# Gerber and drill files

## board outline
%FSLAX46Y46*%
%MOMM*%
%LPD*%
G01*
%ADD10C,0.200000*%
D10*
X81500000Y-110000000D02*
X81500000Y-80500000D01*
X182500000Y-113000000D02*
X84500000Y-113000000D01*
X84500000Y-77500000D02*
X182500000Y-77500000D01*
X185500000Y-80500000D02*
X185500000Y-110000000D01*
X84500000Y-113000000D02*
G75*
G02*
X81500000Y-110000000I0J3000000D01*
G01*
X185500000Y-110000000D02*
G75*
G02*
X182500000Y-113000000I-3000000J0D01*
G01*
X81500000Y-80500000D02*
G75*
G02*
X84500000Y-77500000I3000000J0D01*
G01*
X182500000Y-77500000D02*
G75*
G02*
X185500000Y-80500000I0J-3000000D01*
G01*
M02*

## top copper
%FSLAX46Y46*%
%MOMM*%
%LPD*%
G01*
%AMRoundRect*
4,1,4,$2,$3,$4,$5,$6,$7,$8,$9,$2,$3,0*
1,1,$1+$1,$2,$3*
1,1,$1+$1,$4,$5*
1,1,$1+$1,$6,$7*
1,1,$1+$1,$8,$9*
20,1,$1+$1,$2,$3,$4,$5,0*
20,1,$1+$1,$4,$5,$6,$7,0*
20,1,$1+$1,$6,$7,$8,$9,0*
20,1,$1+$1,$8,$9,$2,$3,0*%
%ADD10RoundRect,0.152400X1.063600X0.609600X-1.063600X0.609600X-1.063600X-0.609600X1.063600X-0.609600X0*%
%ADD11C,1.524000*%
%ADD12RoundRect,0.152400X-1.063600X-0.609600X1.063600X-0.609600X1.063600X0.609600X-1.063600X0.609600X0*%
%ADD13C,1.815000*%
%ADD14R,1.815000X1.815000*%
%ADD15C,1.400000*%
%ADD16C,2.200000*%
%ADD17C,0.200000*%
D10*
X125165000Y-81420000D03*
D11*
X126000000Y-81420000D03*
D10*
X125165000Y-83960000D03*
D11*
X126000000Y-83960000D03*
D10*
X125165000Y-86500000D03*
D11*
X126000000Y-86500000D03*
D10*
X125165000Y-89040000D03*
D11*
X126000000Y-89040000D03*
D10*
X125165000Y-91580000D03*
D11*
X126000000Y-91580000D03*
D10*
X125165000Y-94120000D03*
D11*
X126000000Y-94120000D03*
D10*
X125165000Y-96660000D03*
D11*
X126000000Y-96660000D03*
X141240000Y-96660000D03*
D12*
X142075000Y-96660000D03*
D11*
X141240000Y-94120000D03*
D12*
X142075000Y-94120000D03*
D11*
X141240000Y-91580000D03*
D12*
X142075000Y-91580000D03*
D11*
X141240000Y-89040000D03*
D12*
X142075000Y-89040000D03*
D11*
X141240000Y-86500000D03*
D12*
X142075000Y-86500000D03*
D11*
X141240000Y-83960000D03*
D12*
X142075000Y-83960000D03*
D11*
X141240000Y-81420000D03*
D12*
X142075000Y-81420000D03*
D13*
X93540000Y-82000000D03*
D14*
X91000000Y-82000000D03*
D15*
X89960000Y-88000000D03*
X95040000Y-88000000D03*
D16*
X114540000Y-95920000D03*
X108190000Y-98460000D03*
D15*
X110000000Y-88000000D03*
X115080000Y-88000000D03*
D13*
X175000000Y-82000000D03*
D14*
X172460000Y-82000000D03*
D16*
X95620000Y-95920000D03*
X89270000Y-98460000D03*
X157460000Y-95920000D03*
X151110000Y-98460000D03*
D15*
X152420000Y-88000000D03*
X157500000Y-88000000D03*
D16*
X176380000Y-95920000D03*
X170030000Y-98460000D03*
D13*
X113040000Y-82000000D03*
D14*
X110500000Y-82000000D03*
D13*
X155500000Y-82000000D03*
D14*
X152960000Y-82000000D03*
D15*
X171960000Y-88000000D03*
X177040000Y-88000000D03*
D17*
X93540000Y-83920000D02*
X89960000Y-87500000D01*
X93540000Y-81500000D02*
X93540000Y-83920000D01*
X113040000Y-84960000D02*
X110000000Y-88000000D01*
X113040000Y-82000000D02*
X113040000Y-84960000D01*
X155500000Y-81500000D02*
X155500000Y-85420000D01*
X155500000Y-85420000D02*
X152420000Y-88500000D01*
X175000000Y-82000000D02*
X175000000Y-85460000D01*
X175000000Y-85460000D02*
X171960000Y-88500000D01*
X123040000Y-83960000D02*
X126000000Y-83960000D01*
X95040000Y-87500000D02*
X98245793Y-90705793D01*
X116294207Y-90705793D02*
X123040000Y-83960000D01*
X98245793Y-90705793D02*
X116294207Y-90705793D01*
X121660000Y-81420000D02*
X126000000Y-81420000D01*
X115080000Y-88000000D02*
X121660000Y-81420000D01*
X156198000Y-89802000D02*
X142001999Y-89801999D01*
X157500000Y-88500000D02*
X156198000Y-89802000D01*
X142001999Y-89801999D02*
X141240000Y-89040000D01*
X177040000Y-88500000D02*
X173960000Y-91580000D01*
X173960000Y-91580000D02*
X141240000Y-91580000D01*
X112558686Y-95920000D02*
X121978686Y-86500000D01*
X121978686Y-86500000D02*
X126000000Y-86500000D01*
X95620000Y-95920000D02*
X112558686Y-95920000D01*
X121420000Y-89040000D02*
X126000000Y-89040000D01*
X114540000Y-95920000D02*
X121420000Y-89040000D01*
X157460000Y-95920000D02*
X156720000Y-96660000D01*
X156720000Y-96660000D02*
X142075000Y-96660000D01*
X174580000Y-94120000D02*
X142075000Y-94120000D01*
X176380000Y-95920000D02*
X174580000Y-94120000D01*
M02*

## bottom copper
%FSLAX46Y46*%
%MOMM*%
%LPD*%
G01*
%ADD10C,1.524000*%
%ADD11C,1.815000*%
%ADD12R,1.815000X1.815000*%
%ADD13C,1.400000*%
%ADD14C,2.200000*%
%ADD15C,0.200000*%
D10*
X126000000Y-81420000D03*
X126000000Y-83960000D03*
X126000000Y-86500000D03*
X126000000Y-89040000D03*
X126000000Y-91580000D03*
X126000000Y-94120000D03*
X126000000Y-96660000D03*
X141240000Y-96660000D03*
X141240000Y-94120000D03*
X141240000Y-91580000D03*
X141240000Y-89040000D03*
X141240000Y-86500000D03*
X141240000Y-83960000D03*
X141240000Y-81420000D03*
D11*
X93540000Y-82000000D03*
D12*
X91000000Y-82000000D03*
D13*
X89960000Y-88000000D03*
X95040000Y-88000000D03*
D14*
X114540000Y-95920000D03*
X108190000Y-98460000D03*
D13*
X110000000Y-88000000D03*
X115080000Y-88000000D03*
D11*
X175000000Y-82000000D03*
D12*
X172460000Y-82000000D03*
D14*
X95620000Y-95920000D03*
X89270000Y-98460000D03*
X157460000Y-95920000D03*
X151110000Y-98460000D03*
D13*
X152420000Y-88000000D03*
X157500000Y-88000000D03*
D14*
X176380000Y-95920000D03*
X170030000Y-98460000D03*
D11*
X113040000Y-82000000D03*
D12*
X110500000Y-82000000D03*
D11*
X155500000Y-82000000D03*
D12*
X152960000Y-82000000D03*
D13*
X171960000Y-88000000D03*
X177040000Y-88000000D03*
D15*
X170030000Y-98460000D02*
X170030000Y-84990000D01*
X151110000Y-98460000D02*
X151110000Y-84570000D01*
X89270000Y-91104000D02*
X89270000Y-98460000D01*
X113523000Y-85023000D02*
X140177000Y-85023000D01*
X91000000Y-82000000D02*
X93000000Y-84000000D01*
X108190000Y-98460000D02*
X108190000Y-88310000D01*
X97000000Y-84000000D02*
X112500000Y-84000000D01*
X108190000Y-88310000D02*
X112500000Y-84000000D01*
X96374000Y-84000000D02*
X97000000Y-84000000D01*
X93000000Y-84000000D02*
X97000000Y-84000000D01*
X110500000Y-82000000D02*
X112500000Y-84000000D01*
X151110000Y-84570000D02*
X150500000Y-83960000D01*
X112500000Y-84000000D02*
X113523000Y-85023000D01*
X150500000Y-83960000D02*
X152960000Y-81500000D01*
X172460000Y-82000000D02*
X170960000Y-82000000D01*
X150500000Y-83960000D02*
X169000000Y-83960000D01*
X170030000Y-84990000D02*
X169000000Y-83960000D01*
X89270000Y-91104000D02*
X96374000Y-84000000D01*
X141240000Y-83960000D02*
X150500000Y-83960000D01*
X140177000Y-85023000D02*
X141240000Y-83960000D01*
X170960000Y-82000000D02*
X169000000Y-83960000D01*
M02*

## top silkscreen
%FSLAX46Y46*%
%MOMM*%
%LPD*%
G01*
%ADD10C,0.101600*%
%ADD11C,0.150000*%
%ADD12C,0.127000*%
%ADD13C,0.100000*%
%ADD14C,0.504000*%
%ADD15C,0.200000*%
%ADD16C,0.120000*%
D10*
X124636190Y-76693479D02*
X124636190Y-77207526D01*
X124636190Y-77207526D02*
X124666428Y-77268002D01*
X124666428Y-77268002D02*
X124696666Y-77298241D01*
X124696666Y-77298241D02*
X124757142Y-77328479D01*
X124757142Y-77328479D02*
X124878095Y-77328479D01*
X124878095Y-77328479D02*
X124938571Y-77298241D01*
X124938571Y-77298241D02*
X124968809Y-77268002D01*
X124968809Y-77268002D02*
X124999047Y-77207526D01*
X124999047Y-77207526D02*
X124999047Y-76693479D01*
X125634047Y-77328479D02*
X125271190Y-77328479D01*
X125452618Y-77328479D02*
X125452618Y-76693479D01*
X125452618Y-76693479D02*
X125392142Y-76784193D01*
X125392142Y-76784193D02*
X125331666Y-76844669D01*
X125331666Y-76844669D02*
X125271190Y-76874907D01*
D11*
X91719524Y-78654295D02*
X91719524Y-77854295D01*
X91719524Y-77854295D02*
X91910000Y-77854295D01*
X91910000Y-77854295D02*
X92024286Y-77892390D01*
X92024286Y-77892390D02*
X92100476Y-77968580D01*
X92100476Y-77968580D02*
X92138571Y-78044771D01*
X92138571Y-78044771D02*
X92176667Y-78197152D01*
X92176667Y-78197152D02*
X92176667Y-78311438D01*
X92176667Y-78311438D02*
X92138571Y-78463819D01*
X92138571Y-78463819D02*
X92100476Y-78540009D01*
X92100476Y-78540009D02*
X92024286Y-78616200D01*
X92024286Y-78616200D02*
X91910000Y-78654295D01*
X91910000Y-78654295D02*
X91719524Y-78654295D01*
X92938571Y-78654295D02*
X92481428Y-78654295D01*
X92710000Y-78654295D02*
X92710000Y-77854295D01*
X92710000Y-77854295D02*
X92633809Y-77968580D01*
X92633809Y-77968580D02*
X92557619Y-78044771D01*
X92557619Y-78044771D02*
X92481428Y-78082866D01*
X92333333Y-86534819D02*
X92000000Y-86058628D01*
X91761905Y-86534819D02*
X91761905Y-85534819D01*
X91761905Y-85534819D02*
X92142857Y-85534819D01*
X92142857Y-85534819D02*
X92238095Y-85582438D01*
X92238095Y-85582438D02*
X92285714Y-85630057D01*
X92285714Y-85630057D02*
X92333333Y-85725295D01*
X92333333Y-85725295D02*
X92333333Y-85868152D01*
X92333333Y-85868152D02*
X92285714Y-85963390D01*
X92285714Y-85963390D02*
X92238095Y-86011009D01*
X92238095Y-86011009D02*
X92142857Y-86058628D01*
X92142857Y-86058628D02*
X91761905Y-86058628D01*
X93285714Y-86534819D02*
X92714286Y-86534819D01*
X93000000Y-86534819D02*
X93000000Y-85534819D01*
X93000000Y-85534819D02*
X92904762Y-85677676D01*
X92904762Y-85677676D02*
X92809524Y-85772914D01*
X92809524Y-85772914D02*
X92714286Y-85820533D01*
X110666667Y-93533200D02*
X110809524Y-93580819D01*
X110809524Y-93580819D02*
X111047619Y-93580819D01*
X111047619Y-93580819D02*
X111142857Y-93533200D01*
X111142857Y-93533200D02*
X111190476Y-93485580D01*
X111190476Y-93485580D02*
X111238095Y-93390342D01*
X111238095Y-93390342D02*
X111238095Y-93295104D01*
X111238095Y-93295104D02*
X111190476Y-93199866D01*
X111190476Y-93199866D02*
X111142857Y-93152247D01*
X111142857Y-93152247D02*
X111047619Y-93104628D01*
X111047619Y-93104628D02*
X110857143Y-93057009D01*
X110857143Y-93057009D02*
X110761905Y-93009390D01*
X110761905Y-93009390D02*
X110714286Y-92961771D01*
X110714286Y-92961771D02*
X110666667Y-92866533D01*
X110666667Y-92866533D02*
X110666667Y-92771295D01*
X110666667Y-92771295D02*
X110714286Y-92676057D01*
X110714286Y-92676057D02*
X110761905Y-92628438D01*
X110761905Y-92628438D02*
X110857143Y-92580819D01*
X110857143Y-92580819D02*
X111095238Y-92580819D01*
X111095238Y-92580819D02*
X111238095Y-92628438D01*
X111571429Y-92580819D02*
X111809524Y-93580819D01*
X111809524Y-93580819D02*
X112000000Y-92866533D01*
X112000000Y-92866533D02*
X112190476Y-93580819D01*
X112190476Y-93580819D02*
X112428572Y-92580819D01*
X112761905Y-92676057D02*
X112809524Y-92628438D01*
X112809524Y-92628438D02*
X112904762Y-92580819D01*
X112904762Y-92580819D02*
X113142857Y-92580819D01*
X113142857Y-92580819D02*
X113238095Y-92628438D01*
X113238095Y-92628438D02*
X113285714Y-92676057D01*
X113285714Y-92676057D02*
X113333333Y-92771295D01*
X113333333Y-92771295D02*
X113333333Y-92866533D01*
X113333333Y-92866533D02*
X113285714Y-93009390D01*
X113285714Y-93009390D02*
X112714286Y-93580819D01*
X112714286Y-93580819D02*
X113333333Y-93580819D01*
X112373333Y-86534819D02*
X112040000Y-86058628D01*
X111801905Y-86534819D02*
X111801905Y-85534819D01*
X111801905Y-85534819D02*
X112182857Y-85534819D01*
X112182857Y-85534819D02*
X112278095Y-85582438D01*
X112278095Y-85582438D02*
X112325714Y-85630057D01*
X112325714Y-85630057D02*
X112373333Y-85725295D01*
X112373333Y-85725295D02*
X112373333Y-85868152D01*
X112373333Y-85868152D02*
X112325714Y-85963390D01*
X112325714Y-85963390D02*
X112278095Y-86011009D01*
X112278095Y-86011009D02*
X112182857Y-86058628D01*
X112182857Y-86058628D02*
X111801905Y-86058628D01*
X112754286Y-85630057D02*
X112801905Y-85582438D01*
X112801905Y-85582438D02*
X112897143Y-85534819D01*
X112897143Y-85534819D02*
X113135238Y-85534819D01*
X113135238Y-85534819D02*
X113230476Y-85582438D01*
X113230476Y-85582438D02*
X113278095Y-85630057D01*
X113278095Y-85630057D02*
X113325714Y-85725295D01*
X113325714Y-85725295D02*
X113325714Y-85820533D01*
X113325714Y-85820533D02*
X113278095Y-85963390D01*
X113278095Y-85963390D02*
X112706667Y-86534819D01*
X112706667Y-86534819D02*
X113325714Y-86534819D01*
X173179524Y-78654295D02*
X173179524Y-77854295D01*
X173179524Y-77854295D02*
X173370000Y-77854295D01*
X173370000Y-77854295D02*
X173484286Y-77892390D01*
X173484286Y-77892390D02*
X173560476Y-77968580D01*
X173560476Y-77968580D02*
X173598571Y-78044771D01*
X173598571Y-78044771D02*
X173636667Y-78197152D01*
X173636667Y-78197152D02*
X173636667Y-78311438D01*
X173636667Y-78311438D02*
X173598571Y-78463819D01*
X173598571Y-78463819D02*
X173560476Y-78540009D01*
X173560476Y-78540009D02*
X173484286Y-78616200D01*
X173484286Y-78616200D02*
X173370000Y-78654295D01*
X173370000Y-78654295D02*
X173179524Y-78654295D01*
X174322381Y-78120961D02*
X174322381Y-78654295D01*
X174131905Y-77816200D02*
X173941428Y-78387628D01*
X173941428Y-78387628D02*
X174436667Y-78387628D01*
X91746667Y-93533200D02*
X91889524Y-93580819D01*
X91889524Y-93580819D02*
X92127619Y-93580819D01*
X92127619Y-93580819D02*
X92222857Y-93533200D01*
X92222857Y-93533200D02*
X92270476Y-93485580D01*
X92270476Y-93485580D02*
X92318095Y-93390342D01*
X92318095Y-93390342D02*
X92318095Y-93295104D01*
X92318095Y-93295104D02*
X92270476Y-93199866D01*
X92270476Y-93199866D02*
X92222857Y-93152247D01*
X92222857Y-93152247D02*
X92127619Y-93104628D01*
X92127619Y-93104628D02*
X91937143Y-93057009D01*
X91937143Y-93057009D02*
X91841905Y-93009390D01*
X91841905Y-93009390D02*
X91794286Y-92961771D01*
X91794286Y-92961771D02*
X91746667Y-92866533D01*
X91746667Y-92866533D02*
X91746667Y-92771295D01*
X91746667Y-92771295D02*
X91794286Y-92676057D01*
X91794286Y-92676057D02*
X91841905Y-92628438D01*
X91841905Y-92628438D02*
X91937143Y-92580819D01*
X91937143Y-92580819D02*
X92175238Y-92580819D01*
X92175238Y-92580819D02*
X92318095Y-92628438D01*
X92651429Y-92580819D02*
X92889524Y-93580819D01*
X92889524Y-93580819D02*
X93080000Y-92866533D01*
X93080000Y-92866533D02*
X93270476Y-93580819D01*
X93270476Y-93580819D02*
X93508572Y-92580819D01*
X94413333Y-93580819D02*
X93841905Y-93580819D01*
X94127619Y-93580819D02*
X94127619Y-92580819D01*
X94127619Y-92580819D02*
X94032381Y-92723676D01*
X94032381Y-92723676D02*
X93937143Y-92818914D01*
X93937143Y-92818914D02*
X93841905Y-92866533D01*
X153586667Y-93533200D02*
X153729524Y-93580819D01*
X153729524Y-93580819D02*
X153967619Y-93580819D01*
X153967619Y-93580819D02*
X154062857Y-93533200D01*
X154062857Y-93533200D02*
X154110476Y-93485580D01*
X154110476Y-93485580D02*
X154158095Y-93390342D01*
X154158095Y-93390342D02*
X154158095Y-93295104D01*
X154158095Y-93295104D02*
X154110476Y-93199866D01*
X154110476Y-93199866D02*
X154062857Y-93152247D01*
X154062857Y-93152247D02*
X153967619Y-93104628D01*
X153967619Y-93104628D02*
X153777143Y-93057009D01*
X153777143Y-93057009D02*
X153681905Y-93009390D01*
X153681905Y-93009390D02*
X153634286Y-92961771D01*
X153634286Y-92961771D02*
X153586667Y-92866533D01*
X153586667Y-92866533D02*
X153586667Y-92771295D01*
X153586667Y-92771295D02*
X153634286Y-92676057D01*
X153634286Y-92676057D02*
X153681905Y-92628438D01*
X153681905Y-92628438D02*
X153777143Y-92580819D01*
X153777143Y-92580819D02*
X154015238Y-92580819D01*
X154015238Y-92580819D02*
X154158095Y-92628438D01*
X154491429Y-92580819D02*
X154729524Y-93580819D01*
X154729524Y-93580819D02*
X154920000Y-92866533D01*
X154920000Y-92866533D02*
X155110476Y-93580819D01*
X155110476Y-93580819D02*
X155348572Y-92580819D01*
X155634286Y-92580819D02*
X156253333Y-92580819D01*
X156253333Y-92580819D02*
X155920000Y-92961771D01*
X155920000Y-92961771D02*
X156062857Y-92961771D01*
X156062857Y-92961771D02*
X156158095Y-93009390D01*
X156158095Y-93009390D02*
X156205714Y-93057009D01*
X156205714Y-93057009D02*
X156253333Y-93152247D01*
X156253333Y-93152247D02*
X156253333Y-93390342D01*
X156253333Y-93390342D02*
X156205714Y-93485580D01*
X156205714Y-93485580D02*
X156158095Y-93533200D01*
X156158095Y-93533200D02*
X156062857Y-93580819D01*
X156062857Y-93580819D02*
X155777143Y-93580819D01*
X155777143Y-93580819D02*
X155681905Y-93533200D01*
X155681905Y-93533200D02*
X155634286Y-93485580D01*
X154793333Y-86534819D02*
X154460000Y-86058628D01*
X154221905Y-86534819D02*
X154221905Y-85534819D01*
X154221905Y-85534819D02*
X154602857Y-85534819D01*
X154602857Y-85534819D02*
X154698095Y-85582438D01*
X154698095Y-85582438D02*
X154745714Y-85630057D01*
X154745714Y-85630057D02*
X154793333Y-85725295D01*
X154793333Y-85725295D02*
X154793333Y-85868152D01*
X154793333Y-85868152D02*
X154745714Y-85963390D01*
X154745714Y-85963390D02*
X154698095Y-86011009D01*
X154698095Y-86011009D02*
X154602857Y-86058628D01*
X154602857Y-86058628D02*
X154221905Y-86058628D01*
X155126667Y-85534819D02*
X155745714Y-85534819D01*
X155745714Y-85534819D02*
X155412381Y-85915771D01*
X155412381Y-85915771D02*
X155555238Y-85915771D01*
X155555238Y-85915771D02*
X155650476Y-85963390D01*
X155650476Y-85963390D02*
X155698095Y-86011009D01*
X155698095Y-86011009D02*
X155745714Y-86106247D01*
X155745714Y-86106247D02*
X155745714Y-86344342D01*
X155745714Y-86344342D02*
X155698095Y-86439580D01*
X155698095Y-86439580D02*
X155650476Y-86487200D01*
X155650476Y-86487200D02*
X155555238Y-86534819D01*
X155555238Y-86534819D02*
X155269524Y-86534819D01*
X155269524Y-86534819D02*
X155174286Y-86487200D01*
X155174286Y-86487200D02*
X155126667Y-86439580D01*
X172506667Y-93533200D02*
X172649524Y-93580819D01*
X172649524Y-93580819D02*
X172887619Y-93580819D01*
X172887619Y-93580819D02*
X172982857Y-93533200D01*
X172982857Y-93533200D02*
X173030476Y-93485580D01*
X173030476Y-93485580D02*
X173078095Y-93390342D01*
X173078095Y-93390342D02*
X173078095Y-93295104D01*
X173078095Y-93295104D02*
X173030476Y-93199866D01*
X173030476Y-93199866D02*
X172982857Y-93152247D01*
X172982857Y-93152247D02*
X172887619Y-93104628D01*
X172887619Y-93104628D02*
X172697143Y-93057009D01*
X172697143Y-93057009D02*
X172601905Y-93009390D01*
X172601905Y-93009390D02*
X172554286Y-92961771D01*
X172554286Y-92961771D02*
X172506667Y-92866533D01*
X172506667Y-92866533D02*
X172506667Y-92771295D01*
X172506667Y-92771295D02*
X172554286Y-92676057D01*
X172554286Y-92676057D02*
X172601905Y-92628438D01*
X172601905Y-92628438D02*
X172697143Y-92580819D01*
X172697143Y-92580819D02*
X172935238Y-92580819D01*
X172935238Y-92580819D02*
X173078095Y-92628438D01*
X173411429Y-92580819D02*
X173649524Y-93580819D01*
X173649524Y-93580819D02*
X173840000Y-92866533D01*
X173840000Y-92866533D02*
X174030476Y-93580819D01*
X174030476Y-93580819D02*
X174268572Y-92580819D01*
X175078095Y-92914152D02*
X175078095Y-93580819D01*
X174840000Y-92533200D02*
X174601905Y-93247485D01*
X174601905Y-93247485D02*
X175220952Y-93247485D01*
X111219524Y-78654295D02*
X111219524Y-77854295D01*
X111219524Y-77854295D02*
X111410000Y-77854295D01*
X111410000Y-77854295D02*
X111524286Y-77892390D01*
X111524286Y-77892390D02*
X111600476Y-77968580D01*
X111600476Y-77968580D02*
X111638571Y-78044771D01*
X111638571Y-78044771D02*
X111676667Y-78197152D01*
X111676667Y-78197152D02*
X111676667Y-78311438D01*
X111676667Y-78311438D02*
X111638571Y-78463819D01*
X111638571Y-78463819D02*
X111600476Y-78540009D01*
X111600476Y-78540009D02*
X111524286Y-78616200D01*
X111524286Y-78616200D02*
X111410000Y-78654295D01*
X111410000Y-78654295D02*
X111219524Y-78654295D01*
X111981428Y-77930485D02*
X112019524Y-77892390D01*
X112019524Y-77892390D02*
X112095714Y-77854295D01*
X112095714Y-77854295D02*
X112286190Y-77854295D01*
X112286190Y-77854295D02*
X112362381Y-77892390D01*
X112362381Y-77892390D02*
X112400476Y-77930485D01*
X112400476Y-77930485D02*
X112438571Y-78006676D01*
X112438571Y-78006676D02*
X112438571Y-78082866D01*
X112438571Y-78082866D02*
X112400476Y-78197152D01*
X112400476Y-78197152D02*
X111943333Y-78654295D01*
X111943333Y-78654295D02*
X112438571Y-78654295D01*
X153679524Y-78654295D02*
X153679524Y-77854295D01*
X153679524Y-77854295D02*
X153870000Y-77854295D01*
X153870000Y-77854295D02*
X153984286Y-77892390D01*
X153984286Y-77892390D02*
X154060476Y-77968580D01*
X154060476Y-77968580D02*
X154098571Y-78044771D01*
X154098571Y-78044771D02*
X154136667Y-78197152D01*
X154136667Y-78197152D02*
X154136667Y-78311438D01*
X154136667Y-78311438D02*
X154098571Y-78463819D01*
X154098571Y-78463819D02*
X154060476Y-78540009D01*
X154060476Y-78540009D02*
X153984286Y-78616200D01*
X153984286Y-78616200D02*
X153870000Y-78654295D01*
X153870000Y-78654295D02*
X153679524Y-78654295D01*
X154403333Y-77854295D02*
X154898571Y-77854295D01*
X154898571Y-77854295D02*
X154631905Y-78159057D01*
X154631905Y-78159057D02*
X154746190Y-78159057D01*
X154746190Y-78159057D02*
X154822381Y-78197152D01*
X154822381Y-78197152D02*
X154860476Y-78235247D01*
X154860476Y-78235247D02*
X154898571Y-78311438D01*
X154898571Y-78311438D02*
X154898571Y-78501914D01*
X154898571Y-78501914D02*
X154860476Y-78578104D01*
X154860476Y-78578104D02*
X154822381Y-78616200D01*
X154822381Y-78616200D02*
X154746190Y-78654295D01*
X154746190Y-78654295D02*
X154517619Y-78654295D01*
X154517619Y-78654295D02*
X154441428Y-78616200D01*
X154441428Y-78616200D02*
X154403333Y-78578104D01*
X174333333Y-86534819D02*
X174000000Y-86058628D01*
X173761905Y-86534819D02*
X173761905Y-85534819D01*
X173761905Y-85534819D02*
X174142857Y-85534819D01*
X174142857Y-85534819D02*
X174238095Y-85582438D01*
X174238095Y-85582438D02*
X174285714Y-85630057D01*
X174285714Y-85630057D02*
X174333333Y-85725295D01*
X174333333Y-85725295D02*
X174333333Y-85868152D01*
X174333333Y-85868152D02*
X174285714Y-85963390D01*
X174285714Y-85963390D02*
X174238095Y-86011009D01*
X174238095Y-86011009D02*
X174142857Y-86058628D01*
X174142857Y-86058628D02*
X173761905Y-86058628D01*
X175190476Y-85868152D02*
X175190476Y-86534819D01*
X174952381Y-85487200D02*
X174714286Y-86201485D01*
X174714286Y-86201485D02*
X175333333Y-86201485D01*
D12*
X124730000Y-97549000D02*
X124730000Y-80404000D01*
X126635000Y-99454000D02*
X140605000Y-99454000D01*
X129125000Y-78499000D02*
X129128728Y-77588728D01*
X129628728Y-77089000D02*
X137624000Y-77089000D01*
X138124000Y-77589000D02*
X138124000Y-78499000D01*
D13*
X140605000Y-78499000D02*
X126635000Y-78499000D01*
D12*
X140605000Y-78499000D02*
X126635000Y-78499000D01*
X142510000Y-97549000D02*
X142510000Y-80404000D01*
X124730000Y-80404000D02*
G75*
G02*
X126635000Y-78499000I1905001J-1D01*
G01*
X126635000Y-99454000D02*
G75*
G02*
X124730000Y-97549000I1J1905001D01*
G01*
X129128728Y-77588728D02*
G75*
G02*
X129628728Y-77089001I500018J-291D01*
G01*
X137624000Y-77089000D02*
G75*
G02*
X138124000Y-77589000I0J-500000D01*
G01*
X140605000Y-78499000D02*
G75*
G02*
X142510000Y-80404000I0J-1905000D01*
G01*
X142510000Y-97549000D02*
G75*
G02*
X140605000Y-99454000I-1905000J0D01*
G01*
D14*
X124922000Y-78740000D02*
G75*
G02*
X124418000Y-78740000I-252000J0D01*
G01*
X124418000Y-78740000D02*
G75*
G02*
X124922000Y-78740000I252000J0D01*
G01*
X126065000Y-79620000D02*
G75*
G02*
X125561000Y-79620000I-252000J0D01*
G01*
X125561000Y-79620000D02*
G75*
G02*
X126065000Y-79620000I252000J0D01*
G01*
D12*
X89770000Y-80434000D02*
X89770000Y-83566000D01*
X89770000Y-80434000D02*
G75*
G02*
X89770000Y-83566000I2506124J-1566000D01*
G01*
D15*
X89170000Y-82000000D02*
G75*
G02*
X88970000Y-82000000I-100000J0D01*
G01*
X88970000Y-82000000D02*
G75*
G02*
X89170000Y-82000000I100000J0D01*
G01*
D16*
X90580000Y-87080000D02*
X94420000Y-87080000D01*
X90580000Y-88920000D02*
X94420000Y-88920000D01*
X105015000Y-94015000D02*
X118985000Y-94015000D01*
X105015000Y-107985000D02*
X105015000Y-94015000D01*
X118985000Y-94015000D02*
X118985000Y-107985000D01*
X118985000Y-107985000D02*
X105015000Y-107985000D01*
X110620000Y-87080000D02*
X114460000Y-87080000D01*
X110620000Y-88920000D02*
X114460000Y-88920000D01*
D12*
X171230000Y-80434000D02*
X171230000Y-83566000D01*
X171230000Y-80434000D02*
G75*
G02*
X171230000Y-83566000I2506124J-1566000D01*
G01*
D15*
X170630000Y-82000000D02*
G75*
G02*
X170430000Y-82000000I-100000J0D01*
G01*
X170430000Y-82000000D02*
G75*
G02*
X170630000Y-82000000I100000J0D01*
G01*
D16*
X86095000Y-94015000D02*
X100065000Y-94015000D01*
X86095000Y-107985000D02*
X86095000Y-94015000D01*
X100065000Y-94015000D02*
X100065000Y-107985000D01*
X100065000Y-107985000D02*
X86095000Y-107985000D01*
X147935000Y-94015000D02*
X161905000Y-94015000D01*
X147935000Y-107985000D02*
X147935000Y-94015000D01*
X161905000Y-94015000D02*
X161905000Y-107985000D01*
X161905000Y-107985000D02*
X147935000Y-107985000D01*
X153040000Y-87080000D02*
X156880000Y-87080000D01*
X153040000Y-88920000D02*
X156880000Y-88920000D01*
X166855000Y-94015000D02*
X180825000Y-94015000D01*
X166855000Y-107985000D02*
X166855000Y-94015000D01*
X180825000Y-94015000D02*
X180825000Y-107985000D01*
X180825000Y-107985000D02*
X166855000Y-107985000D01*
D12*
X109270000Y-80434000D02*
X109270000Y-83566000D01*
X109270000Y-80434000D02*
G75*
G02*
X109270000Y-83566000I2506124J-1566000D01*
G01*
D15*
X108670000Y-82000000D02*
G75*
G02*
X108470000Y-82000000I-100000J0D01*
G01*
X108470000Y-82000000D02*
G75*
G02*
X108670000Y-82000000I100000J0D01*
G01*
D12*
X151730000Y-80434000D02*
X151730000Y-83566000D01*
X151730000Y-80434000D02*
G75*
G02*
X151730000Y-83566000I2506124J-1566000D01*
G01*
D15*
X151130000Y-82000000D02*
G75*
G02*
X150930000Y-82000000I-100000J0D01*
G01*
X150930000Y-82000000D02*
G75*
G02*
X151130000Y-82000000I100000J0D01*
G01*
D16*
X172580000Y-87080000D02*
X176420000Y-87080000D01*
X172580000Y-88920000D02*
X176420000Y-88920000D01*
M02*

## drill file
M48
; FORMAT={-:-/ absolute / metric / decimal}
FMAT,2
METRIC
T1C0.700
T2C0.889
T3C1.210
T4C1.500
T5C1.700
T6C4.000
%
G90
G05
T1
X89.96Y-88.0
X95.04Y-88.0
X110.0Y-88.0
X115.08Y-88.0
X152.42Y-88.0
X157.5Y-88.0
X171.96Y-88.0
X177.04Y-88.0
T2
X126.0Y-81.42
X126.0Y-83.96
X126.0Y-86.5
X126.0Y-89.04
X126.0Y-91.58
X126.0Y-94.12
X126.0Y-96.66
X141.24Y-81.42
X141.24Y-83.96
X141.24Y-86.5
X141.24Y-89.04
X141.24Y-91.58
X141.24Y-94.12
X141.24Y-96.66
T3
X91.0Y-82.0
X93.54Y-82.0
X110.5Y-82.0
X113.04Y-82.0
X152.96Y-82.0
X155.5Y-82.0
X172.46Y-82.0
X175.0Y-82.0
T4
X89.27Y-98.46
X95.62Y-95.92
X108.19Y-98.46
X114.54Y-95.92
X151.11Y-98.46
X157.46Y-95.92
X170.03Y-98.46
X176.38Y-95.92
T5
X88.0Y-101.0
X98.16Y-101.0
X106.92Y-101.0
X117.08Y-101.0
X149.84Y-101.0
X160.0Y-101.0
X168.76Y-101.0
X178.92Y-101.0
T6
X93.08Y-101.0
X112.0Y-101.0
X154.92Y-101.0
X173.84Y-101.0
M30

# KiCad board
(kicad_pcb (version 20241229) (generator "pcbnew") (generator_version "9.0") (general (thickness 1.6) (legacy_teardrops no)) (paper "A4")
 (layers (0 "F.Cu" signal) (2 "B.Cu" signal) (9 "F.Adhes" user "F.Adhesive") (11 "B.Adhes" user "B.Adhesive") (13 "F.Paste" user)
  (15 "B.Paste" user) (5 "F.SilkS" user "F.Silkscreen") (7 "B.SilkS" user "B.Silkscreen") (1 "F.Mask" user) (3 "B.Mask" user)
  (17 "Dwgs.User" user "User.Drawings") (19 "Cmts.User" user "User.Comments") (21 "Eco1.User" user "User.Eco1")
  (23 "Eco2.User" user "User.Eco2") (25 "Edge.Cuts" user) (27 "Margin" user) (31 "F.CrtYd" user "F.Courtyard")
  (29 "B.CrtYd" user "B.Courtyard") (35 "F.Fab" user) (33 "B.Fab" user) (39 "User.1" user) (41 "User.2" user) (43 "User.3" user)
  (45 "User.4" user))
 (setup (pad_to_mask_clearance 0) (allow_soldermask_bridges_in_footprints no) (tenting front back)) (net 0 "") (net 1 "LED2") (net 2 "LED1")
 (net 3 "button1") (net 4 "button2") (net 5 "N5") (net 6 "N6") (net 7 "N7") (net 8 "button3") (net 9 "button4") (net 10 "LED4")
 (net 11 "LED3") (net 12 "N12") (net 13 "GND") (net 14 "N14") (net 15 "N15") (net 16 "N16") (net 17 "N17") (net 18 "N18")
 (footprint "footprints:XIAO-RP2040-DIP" (layer "F.Cu") (at 133.62 89.04)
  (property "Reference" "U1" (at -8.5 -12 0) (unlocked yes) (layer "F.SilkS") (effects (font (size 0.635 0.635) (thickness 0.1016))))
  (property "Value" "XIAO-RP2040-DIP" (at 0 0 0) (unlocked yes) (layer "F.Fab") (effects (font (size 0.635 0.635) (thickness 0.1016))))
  (fp_line (start -8.89 8.509) (end -8.89 -8.636) (stroke (width 0.127) (type solid)) (layer "F.SilkS"))
  (fp_line (start -6.985 10.414) (end 6.985 10.414) (stroke (width 0.127) (type solid)) (layer "F.SilkS"))
  (fp_line (start -4.495 -10.541) (end -4.491272 -11.451272) (stroke (width 0.127) (type solid)) (layer "F.SilkS"))
  (fp_line (start -3.991272 -11.951) (end 4.004 -11.951) (stroke (width 0.127) (type solid)) (layer "F.SilkS"))
  (fp_line (start 4.504 -11.451) (end 4.504 -10.541) (stroke (width 0.127) (type solid)) (layer "F.SilkS"))
  (fp_line (start 6.985 -10.541) (end -6.985 -10.541) (stroke (width 0.1) (type solid)) (layer "F.SilkS"))
  (fp_line (start 6.985 -10.541) (end -6.985 -10.541) (stroke (width 0.127) (type solid)) (layer "F.SilkS"))
  (fp_line (start 8.89 8.509) (end 8.89 -8.636) (stroke (width 0.127) (type solid)) (layer "F.SilkS"))
  (fp_arc (start -8.89 -8.636) (mid -8.332038 -9.983038) (end -6.985 -10.541) (stroke (width 0.127) (type solid)) (layer "F.SilkS"))
  (fp_arc (start -6.985 10.414) (mid -8.332038 9.856038) (end -8.89 8.509) (stroke (width 0.127) (type solid)) (layer "F.SilkS"))
  (fp_arc (start -4.491272 -11.451272) (mid -4.344728 -11.80464) (end -3.991272 -11.951) (stroke (width 0.127) (type default))
   (layer "F.SilkS"))
  (fp_arc (start 4.004 -11.951) (mid 4.357553 -11.804553) (end 4.504 -11.451) (stroke (width 0.127) (type default)) (layer "F.SilkS"))
  (fp_arc (start 6.985 -10.541) (mid 8.332038 -9.983038) (end 8.89 -8.636) (stroke (width 0.127) (type solid)) (layer "F.SilkS"))
  (fp_arc (start 8.89 8.509) (mid 8.332038 9.856038) (end 6.985 10.414) (stroke (width 0.127) (type solid)) (layer "F.SilkS"))
  (fp_circle (center -8.95 -10.3) (end -8.95 -10.554) (stroke (width 0.5) (type solid)) (fill yes) (layer "F.SilkS"))
  (fp_circle (center -7.807 -9.42) (end -7.807 -9.674) (stroke (width 0.5) (type solid)) (fill yes) (layer "F.SilkS"))
  (pad "1" smd roundrect (at -8.455 -7.62 180) (size 2.432 1.524) (layers "F.Cu" "F.Mask") (roundrect_rratio 0.1) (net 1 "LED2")
   (thermal_bridge_angle 45))
  (pad "1" thru_hole circle (at -7.62 -7.62 180) (size 1.524 1.524) (drill 0.889) (layers "*.Cu" "*.Mask") (remove_unused_layers no)
   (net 1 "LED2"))
  (pad "2" smd roundrect (at -8.455 -5.08 180) (size 2.432 1.524) (layers "F.Cu" "F.Mask") (roundrect_rratio 0.1) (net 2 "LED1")
   (thermal_bridge_angle 45))
  (pad "2" thru_hole circle (at -7.62 -5.08 180) (size 1.524 1.524) (drill 0.889) (layers "*.Cu" "*.Mask") (remove_unused_layers no)
   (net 2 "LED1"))
  (pad "3" smd roundrect (at -8.455 -2.54 180) (size 2.432 1.524) (layers "F.Cu" "F.Mask") (roundrect_rratio 0.1) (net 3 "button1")
   (thermal_bridge_angle 45))
  (pad "3" thru_hole circle (at -7.62 -2.54 180) (size 1.524 1.524) (drill 0.889) (layers "*.Cu" "*.Mask") (remove_unused_layers no)
   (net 3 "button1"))
  (pad "4" smd roundrect (at -8.455 0 180) (size 2.432 1.524) (layers "F.Cu" "F.Mask") (roundrect_rratio 0.1) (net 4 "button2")
   (thermal_bridge_angle 45))
  (pad "4" thru_hole circle (at -7.62 0 180) (size 1.524 1.524) (drill 0.889) (layers "*.Cu" "*.Mask") (remove_unused_layers no)
   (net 4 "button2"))
  (pad "5" smd roundrect (at -8.455 2.54 180) (size 2.432 1.524) (layers "F.Cu" "F.Mask") (roundrect_rratio 0.1) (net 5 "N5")
   (thermal_bridge_angle 45))
  (pad "5" thru_hole circle (at -7.62 2.54 180) (size 1.524 1.524) (drill 0.889) (layers "*.Cu" "*.Mask") (remove_unused_layers no)
   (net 5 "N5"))
  (pad "6" smd roundrect (at -8.455 5.08 180) (size 2.432 1.524) (layers "F.Cu" "F.Mask") (roundrect_rratio 0.1) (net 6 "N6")
   (thermal_bridge_angle 45))
  (pad "6" thru_hole circle (at -7.62 5.08 180) (size 1.524 1.524) (drill 0.889) (layers "*.Cu" "*.Mask") (remove_unused_layers no)
   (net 6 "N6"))
  (pad "7" smd roundrect (at -8.455 7.62 180) (size 2.432 1.524) (layers "F.Cu" "F.Mask") (roundrect_rratio 0.1) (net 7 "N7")
   (thermal_bridge_angle 45))
  (pad "7" thru_hole circle (at -7.62 7.62 180) (size 1.524 1.524) (drill 0.889) (layers "*.Cu" "*.Mask") (remove_unused_layers no)
   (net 7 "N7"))
  (pad "8" thru_hole circle (at 7.62 7.62) (size 1.524 1.524) (drill 0.889) (layers "*.Cu" "*.Mask") (remove_unused_layers no)
   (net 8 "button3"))
  (pad "8" smd roundrect (at 8.455 7.62) (size 2.432 1.524) (layers "F.Cu" "F.Mask") (roundrect_rratio 0.1) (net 8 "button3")
   (thermal_bridge_angle 45))
  (pad "9" thru_hole circle (at 7.62 5.08) (size 1.524 1.524) (drill 0.889) (layers "*.Cu" "*.Mask") (remove_unused_layers no)
   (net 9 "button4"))
  (pad "9" smd roundrect (at 8.455 5.08) (size 2.432 1.524) (layers "F.Cu" "F.Mask") (roundrect_rratio 0.1) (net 9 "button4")
   (thermal_bridge_angle 45))
  (pad "10" thru_hole circle (at 7.62 2.54) (size 1.524 1.524) (drill 0.889) (layers "*.Cu" "*.Mask") (remove_unused_layers no)
   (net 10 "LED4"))
  (pad "10" smd roundrect (at 8.455 2.54) (size 2.432 1.524) (layers "F.Cu" "F.Mask") (roundrect_rratio 0.1) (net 10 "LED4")
   (thermal_bridge_angle 45))
  (pad "11" thru_hole circle (at 7.62 0) (size 1.524 1.524) (drill 0.889) (layers "*.Cu" "*.Mask") (remove_unused_layers no) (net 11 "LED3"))
  (pad "11" smd roundrect (at 8.455 0) (size 2.432 1.524) (layers "F.Cu" "F.Mask") (roundrect_rratio 0.1) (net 11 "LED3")
   (thermal_bridge_angle 45))
  (pad "12" thru_hole circle (at 7.62 -2.54) (size 1.524 1.524) (drill 0.889) (layers "*.Cu" "*.Mask") (remove_unused_layers no)
   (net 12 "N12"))
  (pad "12" smd roundrect (at 8.455 -2.54) (size 2.432 1.524) (layers "F.Cu" "F.Mask") (roundrect_rratio 0.1) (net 12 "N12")
   (thermal_bridge_angle 45))
  (pad "13" thru_hole circle (at 7.62 -5.08) (size 1.524 1.524) (drill 0.889) (layers "*.Cu" "*.Mask") (remove_unused_layers no)
   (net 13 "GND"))
  (pad "13" smd roundrect (at 8.455 -5.08) (size 2.432 1.524) (layers "F.Cu" "F.Mask") (roundrect_rratio 0.1) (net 13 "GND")
   (thermal_bridge_angle 45))
  (pad "14" thru_hole circle (at 7.62 -7.62) (size 1.524 1.524) (drill 0.889) (layers "*.Cu" "*.Mask") (remove_unused_layers no)
   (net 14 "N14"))
  (pad "14" smd roundrect (at 8.455 -7.62) (size 2.432 1.524) (layers "F.Cu" "F.Mask") (roundrect_rratio 0.1) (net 14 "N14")
   (thermal_bridge_angle 45)))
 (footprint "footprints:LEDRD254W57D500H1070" (layer "F.Cu") (at 92.27 82)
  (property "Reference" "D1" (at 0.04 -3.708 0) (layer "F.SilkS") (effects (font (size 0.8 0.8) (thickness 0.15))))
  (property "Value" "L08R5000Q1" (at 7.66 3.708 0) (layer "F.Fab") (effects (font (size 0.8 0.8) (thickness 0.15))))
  (fp_line (start -2.5 -1.566) (end -2.5 1.566) (stroke (width 0.127) (type solid)) (layer "F.SilkS"))
  (fp_arc (start -2.5 -1.566) (mid 2.961291 0) (end -2.5 1.566) (stroke (width 0.127) (type solid)) (layer "F.SilkS"))
  (fp_circle (center -3.2 0) (end -3.1 0) (stroke (width 0.2) (type solid)) (fill no) (layer "F.SilkS"))
  (pad "A" thru_hole circle (at 1.27 0) (size 1.815 1.815) (drill 1.21) (layers "*.Cu" "*.Mask") (remove_unused_layers no) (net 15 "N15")
   (solder_mask_margin 0.102))
  (pad "C" thru_hole rect (at -1.27 0) (size 1.815 1.815) (drill 1.21) (layers "*.Cu" "*.Mask") (remove_unused_layers no) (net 13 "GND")
   (solder_mask_margin 0.102)))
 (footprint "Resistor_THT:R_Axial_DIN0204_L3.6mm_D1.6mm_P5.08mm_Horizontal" (layer "F.Cu") (at 89.96 88)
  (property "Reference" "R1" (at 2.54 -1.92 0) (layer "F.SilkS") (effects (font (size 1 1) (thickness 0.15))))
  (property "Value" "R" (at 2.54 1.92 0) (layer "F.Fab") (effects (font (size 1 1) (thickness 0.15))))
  (fp_line (start 0.62 -0.92) (end 4.46 -0.92) (stroke (width 0.12) (type solid)) (layer "F.SilkS"))
  (fp_line (start 0.62 0.92) (end 4.46 0.92) (stroke (width 0.12) (type solid)) (layer "F.SilkS"))
  (pad "1" thru_hole circle (at 0 0) (size 1.4 1.4) (drill 0.7) (layers "*.Cu" "*.Mask") (remove_unused_layers no) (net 15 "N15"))
  (pad "2" thru_hole circle (at 5.08 0) (size 1.4 1.4) (drill 0.7) (layers "*.Cu" "*.Mask") (remove_unused_layers no) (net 2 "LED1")))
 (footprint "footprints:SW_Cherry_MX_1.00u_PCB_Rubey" (layer "F.Cu") (at 114.54 95.92)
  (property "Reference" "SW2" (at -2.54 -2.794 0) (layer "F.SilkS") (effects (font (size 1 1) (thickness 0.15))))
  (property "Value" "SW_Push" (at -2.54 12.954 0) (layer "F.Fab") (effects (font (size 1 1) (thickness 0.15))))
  (fp_line (start -9.525 -1.905) (end 4.445 -1.905) (stroke (width 0.12) (type solid)) (layer "F.SilkS"))
  (fp_line (start -9.525 12.065) (end -9.525 -1.905) (stroke (width 0.12) (type solid)) (layer "F.SilkS"))
  (fp_line (start 4.445 -1.905) (end 4.445 12.065) (stroke (width 0.12) (type solid)) (layer "F.SilkS"))
  (fp_line (start 4.445 12.065) (end -9.525 12.065) (stroke (width 0.12) (type solid)) (layer "F.SilkS"))
  (pad "" np_thru_hole circle (at -7.62 5.08) (size 1.7 1.7) (drill 1.7) (layers "*.Cu" "*.Mask"))
  (pad "" np_thru_hole circle (at -2.54 5.08) (size 4 4) (drill 4) (layers "*.Cu" "*.Mask"))
  (pad "" np_thru_hole circle (at 2.54 5.08) (size 1.7 1.7) (drill 1.7) (layers "*.Cu" "*.Mask"))
  (pad "1" thru_hole circle (at 0 0) (size 2.2 2.2) (drill 1.5) (layers "*.Cu" "*.Mask") (remove_unused_layers no) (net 4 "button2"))
  (pad "2" thru_hole circle (at -6.35 2.54) (size 2.2 2.2) (drill 1.5) (layers "*.Cu" "*.Mask") (remove_unused_layers no) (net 13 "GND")))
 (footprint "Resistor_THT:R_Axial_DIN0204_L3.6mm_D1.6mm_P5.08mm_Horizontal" (layer "F.Cu") (at 110 88)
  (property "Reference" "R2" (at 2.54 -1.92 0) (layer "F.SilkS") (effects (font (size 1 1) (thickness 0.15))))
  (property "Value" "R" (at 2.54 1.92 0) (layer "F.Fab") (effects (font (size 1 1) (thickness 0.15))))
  (fp_line (start 0.62 -0.92) (end 4.46 -0.92) (stroke (width 0.12) (type solid)) (layer "F.SilkS"))
  (fp_line (start 0.62 0.92) (end 4.46 0.92) (stroke (width 0.12) (type solid)) (layer "F.SilkS"))
  (pad "1" thru_hole circle (at 0 0) (size 1.4 1.4) (drill 0.7) (layers "*.Cu" "*.Mask") (remove_unused_layers no) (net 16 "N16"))
  (pad "2" thru_hole circle (at 5.08 0) (size 1.4 1.4) (drill 0.7) (layers "*.Cu" "*.Mask") (remove_unused_layers no) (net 1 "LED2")))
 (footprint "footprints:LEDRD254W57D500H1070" (layer "F.Cu") (at 173.73 82)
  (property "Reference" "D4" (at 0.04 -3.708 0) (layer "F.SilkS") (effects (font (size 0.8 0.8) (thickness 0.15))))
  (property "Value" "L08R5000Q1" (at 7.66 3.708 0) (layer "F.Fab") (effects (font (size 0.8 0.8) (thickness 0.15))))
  (fp_line (start -2.5 -1.566) (end -2.5 1.566) (stroke (width 0.127) (type solid)) (layer "F.SilkS"))
  (fp_arc (start -2.5 -1.566) (mid 2.961291 0) (end -2.5 1.566) (stroke (width 0.127) (type solid)) (layer "F.SilkS"))
  (fp_circle (center -3.2 0) (end -3.1 0) (stroke (width 0.2) (type solid)) (fill no) (layer "F.SilkS"))
  (pad "A" thru_hole circle (at 1.27 0) (size 1.815 1.815) (drill 1.21) (layers "*.Cu" "*.Mask") (remove_unused_layers no) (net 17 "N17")
   (solder_mask_margin 0.102))
  (pad "C" thru_hole rect (at -1.27 0) (size 1.815 1.815) (drill 1.21) (layers "*.Cu" "*.Mask") (remove_unused_layers no) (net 13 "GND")
   (solder_mask_margin 0.102)))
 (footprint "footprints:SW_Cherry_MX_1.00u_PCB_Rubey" (layer "F.Cu") (at 95.62 95.92)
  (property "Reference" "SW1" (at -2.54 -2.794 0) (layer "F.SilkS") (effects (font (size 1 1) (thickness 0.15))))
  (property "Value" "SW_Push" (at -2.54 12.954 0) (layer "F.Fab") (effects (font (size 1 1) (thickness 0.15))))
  (fp_line (start -9.525 -1.905) (end 4.445 -1.905) (stroke (width 0.12) (type solid)) (layer "F.SilkS"))
  (fp_line (start -9.525 12.065) (end -9.525 -1.905) (stroke (width 0.12) (type solid)) (layer "F.SilkS"))
  (fp_line (start 4.445 -1.905) (end 4.445 12.065) (stroke (width 0.12) (type solid)) (layer "F.SilkS"))
  (fp_line (start 4.445 12.065) (end -9.525 12.065) (stroke (width 0.12) (type solid)) (layer "F.SilkS"))
  (pad "" np_thru_hole circle (at -7.62 5.08) (size 1.7 1.7) (drill 1.7) (layers "*.Cu" "*.Mask"))
  (pad "" np_thru_hole circle (at -2.54 5.08) (size 4 4) (drill 4) (layers "*.Cu" "*.Mask"))
  (pad "" np_thru_hole circle (at 2.54 5.08) (size 1.7 1.7) (drill 1.7) (layers "*.Cu" "*.Mask"))
  (pad "1" thru_hole circle (at 0 0) (size 2.2 2.2) (drill 1.5) (layers "*.Cu" "*.Mask") (remove_unused_layers no) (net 3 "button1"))
  (pad "2" thru_hole circle (at -6.35 2.54) (size 2.2 2.2) (drill 1.5) (layers "*.Cu" "*.Mask") (remove_unused_layers no) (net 13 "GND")))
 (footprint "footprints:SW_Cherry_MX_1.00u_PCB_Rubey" (layer "F.Cu") (at 157.46 95.92)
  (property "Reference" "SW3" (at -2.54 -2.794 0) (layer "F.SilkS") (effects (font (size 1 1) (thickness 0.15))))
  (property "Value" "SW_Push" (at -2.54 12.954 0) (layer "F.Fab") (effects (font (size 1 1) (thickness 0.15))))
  (fp_line (start -9.525 -1.905) (end 4.445 -1.905) (stroke (width 0.12) (type solid)) (layer "F.SilkS"))
  (fp_line (start -9.525 12.065) (end -9.525 -1.905) (stroke (width 0.12) (type solid)) (layer "F.SilkS"))
  (fp_line (start 4.445 -1.905) (end 4.445 12.065) (stroke (width 0.12) (type solid)) (layer "F.SilkS"))
  (fp_line (start 4.445 12.065) (end -9.525 12.065) (stroke (width 0.12) (type solid)) (layer "F.SilkS"))
  (pad "" np_thru_hole circle (at -7.62 5.08) (size 1.7 1.7) (drill 1.7) (layers "*.Cu" "*.Mask"))
  (pad "" np_thru_hole circle (at -2.54 5.08) (size 4 4) (drill 4) (layers "*.Cu" "*.Mask"))
  (pad "" np_thru_hole circle (at 2.54 5.08) (size 1.7 1.7) (drill 1.7) (layers "*.Cu" "*.Mask"))
  (pad "1" thru_hole circle (at 0 0) (size 2.2 2.2) (drill 1.5) (layers "*.Cu" "*.Mask") (remove_unused_layers no) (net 8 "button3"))
  (pad "2" thru_hole circle (at -6.35 2.54) (size 2.2 2.2) (drill 1.5) (layers "*.Cu" "*.Mask") (remove_unused_layers no) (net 13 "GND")))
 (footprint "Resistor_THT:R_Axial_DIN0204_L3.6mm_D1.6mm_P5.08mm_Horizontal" (layer "F.Cu") (at 152.42 88)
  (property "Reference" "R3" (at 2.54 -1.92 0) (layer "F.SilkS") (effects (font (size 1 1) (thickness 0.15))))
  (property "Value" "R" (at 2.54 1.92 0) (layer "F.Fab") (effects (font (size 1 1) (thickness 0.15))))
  (fp_line (start 0.62 -0.92) (end 4.46 -0.92) (stroke (width 0.12) (type solid)) (layer "F.SilkS"))
  (fp_line (start 0.62 0.92) (end 4.46 0.92) (stroke (width 0.12) (type solid)) (layer "F.SilkS"))
  (pad "1" thru_hole circle (at 0 0) (size 1.4 1.4) (drill 0.7) (layers "*.Cu" "*.Mask") (remove_unused_layers no) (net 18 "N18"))
  (pad "2" thru_hole circle (at 5.08 0) (size 1.4 1.4) (drill 0.7) (layers "*.Cu" "*.Mask") (remove_unused_layers no) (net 11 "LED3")))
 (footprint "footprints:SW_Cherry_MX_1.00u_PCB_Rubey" (layer "F.Cu") (at 176.38 95.92)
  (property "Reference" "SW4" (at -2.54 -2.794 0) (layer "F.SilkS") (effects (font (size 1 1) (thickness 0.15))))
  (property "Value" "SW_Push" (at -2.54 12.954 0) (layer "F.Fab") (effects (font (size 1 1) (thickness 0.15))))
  (fp_line (start -9.525 -1.905) (end 4.445 -1.905) (stroke (width 0.12) (type solid)) (layer "F.SilkS"))
  (fp_line (start -9.525 12.065) (end -9.525 -1.905) (stroke (width 0.12) (type solid)) (layer "F.SilkS"))
  (fp_line (start 4.445 -1.905) (end 4.445 12.065) (stroke (width 0.12) (type solid)) (layer "F.SilkS"))
  (fp_line (start 4.445 12.065) (end -9.525 12.065) (stroke (width 0.12) (type solid)) (layer "F.SilkS"))
  (pad "" np_thru_hole circle (at -7.62 5.08) (size 1.7 1.7) (drill 1.7) (layers "*.Cu" "*.Mask"))
  (pad "" np_thru_hole circle (at -2.54 5.08) (size 4 4) (drill 4) (layers "*.Cu" "*.Mask"))
  (pad "" np_thru_hole circle (at 2.54 5.08) (size 1.7 1.7) (drill 1.7) (layers "*.Cu" "*.Mask"))
  (pad "1" thru_hole circle (at 0 0) (size 2.2 2.2) (drill 1.5) (layers "*.Cu" "*.Mask") (remove_unused_layers no) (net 9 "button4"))
  (pad "2" thru_hole circle (at -6.35 2.54) (size 2.2 2.2) (drill 1.5) (layers "*.Cu" "*.Mask") (remove_unused_layers no) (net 13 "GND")))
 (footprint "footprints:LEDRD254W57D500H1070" (layer "F.Cu") (at 111.77 82)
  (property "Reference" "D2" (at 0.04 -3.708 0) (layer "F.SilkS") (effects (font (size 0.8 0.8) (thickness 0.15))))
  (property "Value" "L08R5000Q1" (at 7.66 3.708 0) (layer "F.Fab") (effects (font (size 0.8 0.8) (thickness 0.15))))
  (fp_line (start -2.5 -1.566) (end -2.5 1.566) (stroke (width 0.127) (type solid)) (layer "F.SilkS"))
  (fp_arc (start -2.5 -1.566) (mid 2.961291 0) (end -2.5 1.566) (stroke (width 0.127) (type solid)) (layer "F.SilkS"))
  (fp_circle (center -3.2 0) (end -3.1 0) (stroke (width 0.2) (type solid)) (fill no) (layer "F.SilkS"))
  (pad "A" thru_hole circle (at 1.27 0) (size 1.815 1.815) (drill 1.21) (layers "*.Cu" "*.Mask") (remove_unused_layers no) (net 16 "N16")
   (solder_mask_margin 0.102))
  (pad "C" thru_hole rect (at -1.27 0) (size 1.815 1.815) (drill 1.21) (layers "*.Cu" "*.Mask") (remove_unused_layers no) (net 13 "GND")
   (solder_mask_margin 0.102)))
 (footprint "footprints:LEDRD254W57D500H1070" (layer "F.Cu") (at 154.23 82)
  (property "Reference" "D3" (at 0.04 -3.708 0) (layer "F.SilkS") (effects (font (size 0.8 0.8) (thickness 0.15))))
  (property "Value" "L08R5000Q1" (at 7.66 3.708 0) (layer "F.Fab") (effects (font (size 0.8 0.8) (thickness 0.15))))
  (fp_line (start -2.5 -1.566) (end -2.5 1.566) (stroke (width 0.127) (type solid)) (layer "F.SilkS"))
  (fp_arc (start -2.5 -1.566) (mid 2.961291 0) (end -2.5 1.566) (stroke (width 0.127) (type solid)) (layer "F.SilkS"))
  (fp_circle (center -3.2 0) (end -3.1 0) (stroke (width 0.2) (type solid)) (fill no) (layer "F.SilkS"))
  (pad "A" thru_hole circle (at 1.27 0) (size 1.815 1.815) (drill 1.21) (layers "*.Cu" "*.Mask") (remove_unused_layers no) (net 18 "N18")
   (solder_mask_margin 0.102))
  (pad "C" thru_hole rect (at -1.27 0) (size 1.815 1.815) (drill 1.21) (layers "*.Cu" "*.Mask") (remove_unused_layers no) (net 13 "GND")
   (solder_mask_margin 0.102)))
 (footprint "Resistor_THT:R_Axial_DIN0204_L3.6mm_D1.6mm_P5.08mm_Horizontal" (layer "F.Cu") (at 171.96 88)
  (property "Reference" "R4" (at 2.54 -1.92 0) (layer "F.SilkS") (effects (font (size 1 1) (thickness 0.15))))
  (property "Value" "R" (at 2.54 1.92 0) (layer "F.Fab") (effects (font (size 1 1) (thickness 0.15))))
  (fp_line (start 0.62 -0.92) (end 4.46 -0.92) (stroke (width 0.12) (type solid)) (layer "F.SilkS"))
  (fp_line (start 0.62 0.92) (end 4.46 0.92) (stroke (width 0.12) (type solid)) (layer "F.SilkS"))
  (pad "1" thru_hole circle (at 0 0) (size 1.4 1.4) (drill 0.7) (layers "*.Cu" "*.Mask") (remove_unused_layers no) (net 17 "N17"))
  (pad "2" thru_hole circle (at 5.08 0) (size 1.4 1.4) (drill 0.7) (layers "*.Cu" "*.Mask") (remove_unused_layers no) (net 10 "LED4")))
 (gr_line (start 81.5 110) (end 81.5 80.5) (stroke (width 0.2) (type default)) (layer "Edge.Cuts"))
 (gr_line (start 182.5 113) (end 84.5 113) (stroke (width 0.2) (type default)) (layer "Edge.Cuts"))
 (gr_line (start 84.5 77.5) (end 182.5 77.5) (stroke (width 0.2) (type default)) (layer "Edge.Cuts"))
 (gr_line (start 185.5 80.5) (end 185.5 110) (stroke (width 0.2) (type default)) (layer "Edge.Cuts"))
 (gr_arc (start 84.5 113) (mid 82.37868 112.12132) (end 81.5 110) (stroke (width 0.2) (type default)) (layer "Edge.Cuts"))
 (gr_arc (start 185.5 110) (mid 184.62132 112.12132) (end 182.5 113) (stroke (width 0.2) (type default)) (layer "Edge.Cuts"))
 (gr_arc (start 81.5 80.5) (mid 82.37868 78.37868) (end 84.5 77.5) (stroke (width 0.2) (type default)) (layer "Edge.Cuts"))
 (gr_arc (start 182.5 77.5) (mid 184.62132 78.37868) (end 185.5 80.5) (stroke (width 0.2) (type default)) (layer "Edge.Cuts"))
 (segment (start 170.03 98.46) (end 170.03 84.99) (width 0.2) (layer "B.Cu") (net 13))
 (segment (start 151.11 98.46) (end 151.11 84.57) (width 0.2) (layer "B.Cu") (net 13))
 (segment (start 89.27 91.104) (end 89.27 98.46) (width 0.2) (layer "B.Cu") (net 13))
 (segment (start 113.523 85.023) (end 140.177 85.023) (width 0.2) (layer "B.Cu") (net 13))
 (segment (start 91 82) (end 93 84) (width 0.2) (layer "B.Cu") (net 13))
 (segment (start 108.19 98.46) (end 108.19 88.31) (width 0.2) (layer "B.Cu") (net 13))
 (segment (start 97 84) (end 112.5 84) (width 0.2) (layer "B.Cu") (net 13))
 (segment (start 108.19 88.31) (end 112.5 84) (width 0.2) (layer "B.Cu") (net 13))
 (segment (start 96.374 84) (end 97 84) (width 0.2) (layer "B.Cu") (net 13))
 (segment (start 93 84) (end 97 84) (width 0.2) (layer "B.Cu") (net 13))
 (segment (start 110.5 82) (end 112.5 84) (width 0.2) (layer "B.Cu") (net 13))
 (segment (start 151.11 84.57) (end 150.5 83.96) (width 0.2) (layer "B.Cu") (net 13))
 (segment (start 112.5 84) (end 113.523 85.023) (width 0.2) (layer "B.Cu") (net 13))
 (segment (start 150.5 83.96) (end 152.96 81.5) (width 0.2) (layer "B.Cu") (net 13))
 (segment (start 172.46 82) (end 170.96 82) (width 0.2) (layer "B.Cu") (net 13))
 (segment (start 150.5 83.96) (end 169 83.96) (width 0.2) (layer "B.Cu") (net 13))
 (segment (start 170.03 84.99) (end 169 83.96) (width 0.2) (layer "B.Cu") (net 13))
 (segment (start 89.27 91.104) (end 96.374 84) (width 0.2) (layer "B.Cu") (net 13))
 (segment (start 141.24 83.96) (end 150.5 83.96) (width 0.2) (layer "B.Cu") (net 13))
 (segment (start 140.177 85.023) (end 141.24 83.96) (width 0.2) (layer "B.Cu") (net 13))
 (segment (start 170.96 82) (end 169 83.96) (width 0.2) (layer "B.Cu") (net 13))
 (segment (start 93.54 83.92) (end 89.96 87.5) (width 0.2) (layer "F.Cu") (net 15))
 (segment (start 93.54 81.5) (end 93.54 83.92) (width 0.2) (layer "F.Cu") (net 15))
 (segment (start 113.04 84.96) (end 110 88) (width 0.2) (layer "F.Cu") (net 16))
 (segment (start 113.04 82) (end 113.04 84.96) (width 0.2) (layer "F.Cu") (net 16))
 (segment (start 155.5 81.5) (end 155.5 85.42) (width 0.2) (layer "F.Cu") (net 18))
 (segment (start 155.5 85.42) (end 152.42 88.5) (width 0.2) (layer "F.Cu") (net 18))
 (segment (start 175 82) (end 175 85.46) (width 0.2) (layer "F.Cu") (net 17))
 (segment (start 175 85.46) (end 171.96 88.5) (width 0.2) (layer "F.Cu") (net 17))
 (segment (start 123.04 83.96) (end 126 83.96) (width 0.2) (layer "F.Cu") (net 2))
 (segment (start 95.04 87.5) (end 98.245793 90.705793) (width 0.2) (layer "F.Cu") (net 2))
 (segment (start 116.294207 90.705793) (end 123.04 83.96) (width 0.2) (layer "F.Cu") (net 2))
 (segment (start 98.245793 90.705793) (end 116.294207 90.705793) (width 0.2) (layer "F.Cu") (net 2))
 (segment (start 121.66 81.42) (end 126 81.42) (width 0.2) (layer "F.Cu") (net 1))
 (segment (start 115.08 88) (end 121.66 81.42) (width 0.2) (layer "F.Cu") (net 1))
 (segment (start 156.198 89.802) (end 142.001999 89.801999) (width 0.2) (layer "F.Cu") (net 11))
 (segment (start 157.5 88.5) (end 156.198 89.802) (width 0.2) (layer "F.Cu") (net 11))
 (segment (start 142.001999 89.801999) (end 141.24 89.04) (width 0.2) (layer "F.Cu") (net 11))
 (segment (start 177.04 88.5) (end 173.96 91.58) (width 0.2) (layer "F.Cu") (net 10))
 (segment (start 173.96 91.58) (end 141.24 91.58) (width 0.2) (layer "F.Cu") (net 10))
 (segment (start 112.558686 95.92) (end 121.978686 86.5) (width 0.2) (layer "F.Cu") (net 3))
 (segment (start 121.978686 86.5) (end 126 86.5) (width 0.2) (layer "F.Cu") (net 3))
 (segment (start 95.62 95.92) (end 112.558686 95.92) (width 0.2) (layer "F.Cu") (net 3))
 (segment (start 121.42 89.04) (end 126 89.04) (width 0.2) (layer "F.Cu") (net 4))
 (segment (start 114.54 95.92) (end 121.42 89.04) (width 0.2) (layer "F.Cu") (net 4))
 (segment (start 157.46 95.92) (end 156.72 96.66) (width 0.2) (layer "F.Cu") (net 8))
 (segment (start 156.72 96.66) (end 142.075 96.66) (width 0.2) (layer "F.Cu") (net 8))
 (segment (start 174.58 94.12) (end 142.075 94.12) (width 0.2) (layer "F.Cu") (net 9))
 (segment (start 176.38 95.92) (end 174.58 94.12) (width 0.2) (layer "F.Cu") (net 9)))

